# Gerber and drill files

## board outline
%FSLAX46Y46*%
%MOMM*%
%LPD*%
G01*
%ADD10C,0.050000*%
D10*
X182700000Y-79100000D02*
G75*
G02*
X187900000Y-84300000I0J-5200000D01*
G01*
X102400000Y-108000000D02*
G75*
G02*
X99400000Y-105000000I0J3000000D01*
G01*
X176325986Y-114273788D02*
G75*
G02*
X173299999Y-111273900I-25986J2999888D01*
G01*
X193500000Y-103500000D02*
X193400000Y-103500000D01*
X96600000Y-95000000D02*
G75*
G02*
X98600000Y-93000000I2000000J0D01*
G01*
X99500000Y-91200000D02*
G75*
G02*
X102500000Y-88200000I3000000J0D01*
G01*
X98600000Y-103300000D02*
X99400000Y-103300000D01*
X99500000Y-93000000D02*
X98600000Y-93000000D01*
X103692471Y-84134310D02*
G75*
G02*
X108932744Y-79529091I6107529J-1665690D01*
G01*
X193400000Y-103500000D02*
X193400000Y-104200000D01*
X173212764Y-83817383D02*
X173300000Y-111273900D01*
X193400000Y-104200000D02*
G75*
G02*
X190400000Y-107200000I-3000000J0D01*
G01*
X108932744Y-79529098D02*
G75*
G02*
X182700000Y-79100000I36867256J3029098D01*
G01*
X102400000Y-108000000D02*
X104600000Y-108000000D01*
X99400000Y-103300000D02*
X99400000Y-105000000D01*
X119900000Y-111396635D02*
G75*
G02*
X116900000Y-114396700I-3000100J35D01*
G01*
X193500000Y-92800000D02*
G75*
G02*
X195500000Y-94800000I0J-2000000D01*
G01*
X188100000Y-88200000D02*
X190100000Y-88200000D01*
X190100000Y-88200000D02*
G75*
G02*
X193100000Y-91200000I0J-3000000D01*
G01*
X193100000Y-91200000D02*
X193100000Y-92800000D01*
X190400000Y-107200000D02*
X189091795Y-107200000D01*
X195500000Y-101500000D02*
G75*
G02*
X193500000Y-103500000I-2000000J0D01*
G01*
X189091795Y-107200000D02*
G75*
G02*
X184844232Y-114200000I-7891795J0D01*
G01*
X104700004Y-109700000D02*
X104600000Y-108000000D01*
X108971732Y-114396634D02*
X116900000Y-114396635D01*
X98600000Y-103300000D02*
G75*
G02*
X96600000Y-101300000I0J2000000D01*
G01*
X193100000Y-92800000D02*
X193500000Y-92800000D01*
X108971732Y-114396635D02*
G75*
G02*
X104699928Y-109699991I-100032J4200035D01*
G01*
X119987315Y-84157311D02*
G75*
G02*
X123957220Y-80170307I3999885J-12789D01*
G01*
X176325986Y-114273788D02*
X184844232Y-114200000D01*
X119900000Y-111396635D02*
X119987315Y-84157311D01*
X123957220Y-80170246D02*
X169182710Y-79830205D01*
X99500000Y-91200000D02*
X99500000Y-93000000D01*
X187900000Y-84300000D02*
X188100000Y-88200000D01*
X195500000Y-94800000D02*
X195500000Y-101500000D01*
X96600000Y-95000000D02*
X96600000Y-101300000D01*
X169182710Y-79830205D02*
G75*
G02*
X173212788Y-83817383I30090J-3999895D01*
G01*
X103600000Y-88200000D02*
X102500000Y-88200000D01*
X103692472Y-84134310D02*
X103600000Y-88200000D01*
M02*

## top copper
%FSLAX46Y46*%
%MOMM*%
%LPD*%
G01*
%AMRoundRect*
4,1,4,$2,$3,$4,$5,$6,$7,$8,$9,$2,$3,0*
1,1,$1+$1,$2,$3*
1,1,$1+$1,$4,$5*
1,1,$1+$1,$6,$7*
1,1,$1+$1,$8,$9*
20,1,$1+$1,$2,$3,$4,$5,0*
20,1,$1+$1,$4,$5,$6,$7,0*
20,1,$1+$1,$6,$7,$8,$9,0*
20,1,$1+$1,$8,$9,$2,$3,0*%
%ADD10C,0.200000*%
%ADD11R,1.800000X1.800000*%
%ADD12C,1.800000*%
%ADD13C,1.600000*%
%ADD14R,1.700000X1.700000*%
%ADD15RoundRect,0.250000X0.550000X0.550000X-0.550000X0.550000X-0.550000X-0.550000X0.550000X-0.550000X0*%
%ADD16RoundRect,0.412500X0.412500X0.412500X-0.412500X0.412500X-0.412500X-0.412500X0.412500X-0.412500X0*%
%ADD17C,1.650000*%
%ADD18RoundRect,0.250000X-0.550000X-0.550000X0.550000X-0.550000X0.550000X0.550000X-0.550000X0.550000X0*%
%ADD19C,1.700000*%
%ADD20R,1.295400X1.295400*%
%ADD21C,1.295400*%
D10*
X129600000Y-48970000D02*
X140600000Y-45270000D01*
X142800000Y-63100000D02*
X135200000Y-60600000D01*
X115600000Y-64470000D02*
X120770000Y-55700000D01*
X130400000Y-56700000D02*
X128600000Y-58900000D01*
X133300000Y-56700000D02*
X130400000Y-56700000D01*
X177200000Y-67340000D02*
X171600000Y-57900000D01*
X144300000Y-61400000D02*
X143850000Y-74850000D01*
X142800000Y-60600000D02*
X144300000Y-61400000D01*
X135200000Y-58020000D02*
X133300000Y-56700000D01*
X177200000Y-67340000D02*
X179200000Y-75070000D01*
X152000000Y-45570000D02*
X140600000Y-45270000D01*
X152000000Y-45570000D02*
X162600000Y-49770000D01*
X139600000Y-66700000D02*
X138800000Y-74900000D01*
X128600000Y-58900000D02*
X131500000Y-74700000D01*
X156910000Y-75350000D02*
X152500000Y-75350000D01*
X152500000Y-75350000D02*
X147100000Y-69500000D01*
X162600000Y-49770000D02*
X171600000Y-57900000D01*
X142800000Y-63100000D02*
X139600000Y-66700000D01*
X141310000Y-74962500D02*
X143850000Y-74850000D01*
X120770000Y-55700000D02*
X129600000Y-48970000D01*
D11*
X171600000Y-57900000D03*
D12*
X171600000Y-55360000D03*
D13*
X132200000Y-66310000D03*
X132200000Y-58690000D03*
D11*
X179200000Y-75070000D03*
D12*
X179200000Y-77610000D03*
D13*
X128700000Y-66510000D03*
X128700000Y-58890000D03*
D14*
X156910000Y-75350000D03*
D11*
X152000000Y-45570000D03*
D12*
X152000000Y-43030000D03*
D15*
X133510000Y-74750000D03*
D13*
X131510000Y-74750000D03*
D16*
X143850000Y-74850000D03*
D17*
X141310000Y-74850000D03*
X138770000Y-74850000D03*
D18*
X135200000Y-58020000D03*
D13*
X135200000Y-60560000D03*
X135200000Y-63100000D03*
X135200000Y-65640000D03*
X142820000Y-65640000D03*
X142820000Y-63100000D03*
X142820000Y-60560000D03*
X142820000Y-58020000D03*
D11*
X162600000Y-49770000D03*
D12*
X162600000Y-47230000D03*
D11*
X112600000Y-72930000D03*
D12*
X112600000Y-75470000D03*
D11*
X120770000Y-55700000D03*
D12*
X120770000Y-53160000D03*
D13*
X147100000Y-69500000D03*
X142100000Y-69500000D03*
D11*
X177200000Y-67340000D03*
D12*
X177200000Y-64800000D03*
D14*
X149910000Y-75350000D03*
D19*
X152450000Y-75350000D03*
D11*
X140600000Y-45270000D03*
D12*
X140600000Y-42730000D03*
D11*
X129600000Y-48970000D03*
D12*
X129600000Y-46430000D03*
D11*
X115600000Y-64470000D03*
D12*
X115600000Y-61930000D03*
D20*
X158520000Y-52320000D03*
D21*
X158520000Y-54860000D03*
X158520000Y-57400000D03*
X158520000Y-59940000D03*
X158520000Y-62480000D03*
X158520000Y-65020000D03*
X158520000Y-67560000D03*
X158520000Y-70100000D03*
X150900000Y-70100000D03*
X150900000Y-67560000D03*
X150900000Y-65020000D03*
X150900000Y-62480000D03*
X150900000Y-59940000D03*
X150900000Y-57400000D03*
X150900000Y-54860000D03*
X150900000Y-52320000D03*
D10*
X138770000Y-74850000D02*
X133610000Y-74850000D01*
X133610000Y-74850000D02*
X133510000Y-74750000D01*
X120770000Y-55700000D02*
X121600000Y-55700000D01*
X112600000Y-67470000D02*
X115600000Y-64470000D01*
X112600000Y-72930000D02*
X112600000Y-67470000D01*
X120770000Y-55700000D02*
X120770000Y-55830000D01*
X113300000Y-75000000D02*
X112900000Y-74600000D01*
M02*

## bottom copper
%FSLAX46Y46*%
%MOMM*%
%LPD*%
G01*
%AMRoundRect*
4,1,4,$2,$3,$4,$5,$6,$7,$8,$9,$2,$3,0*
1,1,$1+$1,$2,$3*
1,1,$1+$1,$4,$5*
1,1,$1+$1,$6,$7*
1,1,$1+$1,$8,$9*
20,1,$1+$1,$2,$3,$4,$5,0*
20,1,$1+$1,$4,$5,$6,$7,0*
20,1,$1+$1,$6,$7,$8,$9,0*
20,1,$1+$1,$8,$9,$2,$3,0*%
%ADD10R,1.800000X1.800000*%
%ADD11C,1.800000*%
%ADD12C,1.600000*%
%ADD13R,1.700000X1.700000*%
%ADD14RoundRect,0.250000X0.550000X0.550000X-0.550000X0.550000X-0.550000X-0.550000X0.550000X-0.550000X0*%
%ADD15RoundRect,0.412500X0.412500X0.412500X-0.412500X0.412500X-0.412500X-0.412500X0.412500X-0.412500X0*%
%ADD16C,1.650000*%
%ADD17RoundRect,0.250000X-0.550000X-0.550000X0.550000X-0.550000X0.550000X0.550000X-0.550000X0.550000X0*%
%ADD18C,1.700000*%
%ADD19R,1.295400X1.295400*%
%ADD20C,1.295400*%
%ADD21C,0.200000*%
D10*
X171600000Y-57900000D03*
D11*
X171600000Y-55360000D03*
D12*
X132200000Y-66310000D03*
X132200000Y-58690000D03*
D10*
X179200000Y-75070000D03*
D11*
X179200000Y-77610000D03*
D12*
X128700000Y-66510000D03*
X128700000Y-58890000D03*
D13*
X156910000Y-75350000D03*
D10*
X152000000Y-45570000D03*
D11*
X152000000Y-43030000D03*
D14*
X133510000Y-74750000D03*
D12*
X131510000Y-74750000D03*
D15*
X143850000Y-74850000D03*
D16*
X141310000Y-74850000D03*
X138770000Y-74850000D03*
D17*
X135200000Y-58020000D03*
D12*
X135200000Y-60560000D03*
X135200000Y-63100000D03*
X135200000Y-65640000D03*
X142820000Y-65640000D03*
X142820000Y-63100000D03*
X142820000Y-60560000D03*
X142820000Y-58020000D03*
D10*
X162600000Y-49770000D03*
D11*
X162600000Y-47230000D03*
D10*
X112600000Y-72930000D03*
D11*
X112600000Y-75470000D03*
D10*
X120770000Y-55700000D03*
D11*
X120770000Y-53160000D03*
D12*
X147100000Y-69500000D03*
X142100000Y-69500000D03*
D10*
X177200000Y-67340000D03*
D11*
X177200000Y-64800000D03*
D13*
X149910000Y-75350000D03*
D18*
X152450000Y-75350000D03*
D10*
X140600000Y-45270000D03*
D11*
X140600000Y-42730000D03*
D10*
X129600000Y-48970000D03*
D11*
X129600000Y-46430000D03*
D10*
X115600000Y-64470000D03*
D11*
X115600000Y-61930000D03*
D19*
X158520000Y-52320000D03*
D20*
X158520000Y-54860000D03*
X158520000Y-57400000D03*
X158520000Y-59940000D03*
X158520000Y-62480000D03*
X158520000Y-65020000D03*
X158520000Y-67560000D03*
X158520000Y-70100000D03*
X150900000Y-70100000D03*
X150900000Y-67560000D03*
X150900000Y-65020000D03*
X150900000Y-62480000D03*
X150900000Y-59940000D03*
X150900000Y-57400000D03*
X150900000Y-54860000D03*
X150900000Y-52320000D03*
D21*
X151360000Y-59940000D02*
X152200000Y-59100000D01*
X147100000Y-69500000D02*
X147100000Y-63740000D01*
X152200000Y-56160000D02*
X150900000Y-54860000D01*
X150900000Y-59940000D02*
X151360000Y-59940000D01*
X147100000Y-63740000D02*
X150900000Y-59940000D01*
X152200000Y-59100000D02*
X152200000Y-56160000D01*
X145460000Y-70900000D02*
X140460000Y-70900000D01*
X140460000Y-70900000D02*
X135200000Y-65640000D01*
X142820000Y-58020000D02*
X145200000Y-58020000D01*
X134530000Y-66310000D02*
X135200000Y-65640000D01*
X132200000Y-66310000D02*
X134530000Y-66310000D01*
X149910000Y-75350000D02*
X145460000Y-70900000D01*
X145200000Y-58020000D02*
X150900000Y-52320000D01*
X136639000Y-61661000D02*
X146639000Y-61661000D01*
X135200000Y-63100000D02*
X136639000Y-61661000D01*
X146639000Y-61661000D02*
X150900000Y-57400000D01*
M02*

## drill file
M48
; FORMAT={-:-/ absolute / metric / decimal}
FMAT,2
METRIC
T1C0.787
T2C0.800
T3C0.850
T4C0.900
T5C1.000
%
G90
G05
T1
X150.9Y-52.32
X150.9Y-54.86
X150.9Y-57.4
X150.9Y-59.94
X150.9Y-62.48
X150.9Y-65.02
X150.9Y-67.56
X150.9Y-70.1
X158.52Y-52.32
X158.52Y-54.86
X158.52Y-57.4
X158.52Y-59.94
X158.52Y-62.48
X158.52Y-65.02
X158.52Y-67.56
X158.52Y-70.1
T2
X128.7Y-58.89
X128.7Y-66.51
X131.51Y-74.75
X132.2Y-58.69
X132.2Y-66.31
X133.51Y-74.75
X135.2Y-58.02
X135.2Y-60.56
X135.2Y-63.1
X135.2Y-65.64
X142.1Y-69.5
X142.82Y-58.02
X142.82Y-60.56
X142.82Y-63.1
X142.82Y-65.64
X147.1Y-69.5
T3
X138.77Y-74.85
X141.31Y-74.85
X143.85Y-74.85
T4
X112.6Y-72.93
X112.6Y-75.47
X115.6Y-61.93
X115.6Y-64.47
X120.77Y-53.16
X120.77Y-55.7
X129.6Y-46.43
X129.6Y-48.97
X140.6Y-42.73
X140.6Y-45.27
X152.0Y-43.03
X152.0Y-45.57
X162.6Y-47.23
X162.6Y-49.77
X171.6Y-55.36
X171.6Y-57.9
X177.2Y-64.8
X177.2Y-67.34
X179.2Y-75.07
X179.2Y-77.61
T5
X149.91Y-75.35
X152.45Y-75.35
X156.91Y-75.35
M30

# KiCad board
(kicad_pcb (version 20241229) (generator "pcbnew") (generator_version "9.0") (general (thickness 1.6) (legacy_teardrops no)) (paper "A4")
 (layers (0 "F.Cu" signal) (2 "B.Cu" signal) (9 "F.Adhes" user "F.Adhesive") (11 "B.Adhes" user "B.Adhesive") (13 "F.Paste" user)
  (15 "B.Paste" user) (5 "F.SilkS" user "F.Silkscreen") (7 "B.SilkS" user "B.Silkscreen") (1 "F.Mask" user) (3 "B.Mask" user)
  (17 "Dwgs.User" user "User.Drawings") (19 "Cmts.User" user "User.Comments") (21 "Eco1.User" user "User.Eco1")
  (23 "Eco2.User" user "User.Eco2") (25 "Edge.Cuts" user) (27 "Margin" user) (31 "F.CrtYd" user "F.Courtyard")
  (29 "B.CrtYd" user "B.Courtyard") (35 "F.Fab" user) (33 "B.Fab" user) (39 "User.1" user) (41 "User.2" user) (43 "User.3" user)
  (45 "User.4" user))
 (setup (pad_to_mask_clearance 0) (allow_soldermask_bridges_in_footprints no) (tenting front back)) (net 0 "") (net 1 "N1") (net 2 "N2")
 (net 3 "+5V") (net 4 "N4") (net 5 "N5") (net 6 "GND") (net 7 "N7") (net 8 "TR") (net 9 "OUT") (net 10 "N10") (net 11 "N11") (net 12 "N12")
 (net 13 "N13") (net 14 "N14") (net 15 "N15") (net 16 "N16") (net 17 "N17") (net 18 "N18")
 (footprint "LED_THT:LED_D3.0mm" (layer "F.Cu") (at 171.6 57.9 90)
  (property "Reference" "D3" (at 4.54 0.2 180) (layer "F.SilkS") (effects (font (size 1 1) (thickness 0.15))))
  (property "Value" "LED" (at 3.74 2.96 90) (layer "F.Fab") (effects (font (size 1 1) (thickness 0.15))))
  (pad "1" thru_hole rect (at 0 0 90) (size 1.8 1.8) (drill 0.9) (layers "*.Cu" "*.Mask") (remove_unused_layers no) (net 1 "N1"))
  (pad "2" thru_hole circle (at 2.54 0 90) (size 1.8 1.8) (drill 0.9) (layers "*.Cu" "*.Mask") (remove_unused_layers no) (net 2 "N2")))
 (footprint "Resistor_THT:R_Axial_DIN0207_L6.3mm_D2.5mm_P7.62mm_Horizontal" (layer "F.Cu") (at 132.2 66.31 90)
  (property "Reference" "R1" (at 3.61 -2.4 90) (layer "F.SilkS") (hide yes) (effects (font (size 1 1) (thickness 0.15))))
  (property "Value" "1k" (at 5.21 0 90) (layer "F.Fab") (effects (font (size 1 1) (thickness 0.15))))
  (pad "1" thru_hole circle (at 0 0 90) (size 1.6 1.6) (drill 0.8) (layers "*.Cu" "*.Mask") (remove_unused_layers no) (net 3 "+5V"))
  (pad "2" thru_hole circle (at 7.62 0 90) (size 1.6 1.6) (drill 0.8) (layers "*.Cu" "*.Mask") (remove_unused_layers no) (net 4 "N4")))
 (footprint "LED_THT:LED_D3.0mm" (layer "F.Cu") (at 179.2 75.07 -90)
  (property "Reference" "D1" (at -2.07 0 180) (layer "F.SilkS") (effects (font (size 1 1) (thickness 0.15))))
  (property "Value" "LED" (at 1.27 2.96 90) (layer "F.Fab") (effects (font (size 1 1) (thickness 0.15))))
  (pad "1" thru_hole rect (at 0 0 270) (size 1.8 1.8) (drill 0.9) (layers "*.Cu" "*.Mask") (remove_unused_layers no) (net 1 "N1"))
  (pad "2" thru_hole circle (at 2.54 0 270) (size 1.8 1.8) (drill 0.9) (layers "*.Cu" "*.Mask") (remove_unused_layers no) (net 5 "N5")))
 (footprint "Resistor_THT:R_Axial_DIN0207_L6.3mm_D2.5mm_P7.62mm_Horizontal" (layer "F.Cu") (at 128.7 66.51 90)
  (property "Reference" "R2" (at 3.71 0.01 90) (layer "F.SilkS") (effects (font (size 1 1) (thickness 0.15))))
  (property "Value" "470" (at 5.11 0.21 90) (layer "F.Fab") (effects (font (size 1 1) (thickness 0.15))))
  (pad "1" thru_hole circle (at 0 0 90) (size 1.6 1.6) (drill 0.8) (layers "*.Cu" "*.Mask") (remove_unused_layers no) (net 1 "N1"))
  (pad "2" thru_hole circle (at 7.62 0 90) (size 1.6 1.6) (drill 0.8) (layers "*.Cu" "*.Mask") (remove_unused_layers no) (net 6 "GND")))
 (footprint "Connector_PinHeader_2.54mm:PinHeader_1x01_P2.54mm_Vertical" (layer "F.Cu") (at 156.91 75.35)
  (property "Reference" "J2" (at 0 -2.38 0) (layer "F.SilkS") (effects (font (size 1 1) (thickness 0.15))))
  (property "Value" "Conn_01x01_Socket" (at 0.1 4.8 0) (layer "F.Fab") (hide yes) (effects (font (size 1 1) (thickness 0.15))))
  (pad "1" thru_hole rect (at 0 0) (size 1.7 1.7) (drill 1) (layers "*.Cu" "*.Mask") (remove_unused_layers no) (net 6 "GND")))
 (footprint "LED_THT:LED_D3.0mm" (layer "F.Cu") (at 152 45.57 90)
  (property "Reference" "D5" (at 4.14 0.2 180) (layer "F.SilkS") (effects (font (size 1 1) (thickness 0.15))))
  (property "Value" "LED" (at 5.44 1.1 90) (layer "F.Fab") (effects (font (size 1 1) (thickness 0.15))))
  (pad "1" thru_hole rect (at 0 0 90) (size 1.8 1.8) (drill 0.9) (layers "*.Cu" "*.Mask") (remove_unused_layers no) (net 1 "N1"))
  (pad "2" thru_hole circle (at 2.54 0 90) (size 1.8 1.8) (drill 0.9) (layers "*.Cu" "*.Mask") (remove_unused_layers no) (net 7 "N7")))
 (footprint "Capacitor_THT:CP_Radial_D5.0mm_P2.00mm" (layer "F.Cu") (at 133.51 74.75 180)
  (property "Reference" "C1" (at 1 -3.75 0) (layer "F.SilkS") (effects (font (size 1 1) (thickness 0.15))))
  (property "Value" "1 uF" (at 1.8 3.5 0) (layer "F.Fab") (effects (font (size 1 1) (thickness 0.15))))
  (pad "1" thru_hole roundrect (at 0 0 180) (size 1.6 1.6) (drill 0.8) (layers "*.Cu" "*.Mask") (remove_unused_layers no)
   (roundrect_rratio 0.15625) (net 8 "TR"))
  (pad "2" thru_hole circle (at 2 0 180) (size 1.6 1.6) (drill 0.8) (layers "*.Cu" "*.Mask") (remove_unused_layers no) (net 6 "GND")))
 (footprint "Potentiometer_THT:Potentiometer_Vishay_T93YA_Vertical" (layer "F.Cu") (at 143.85 74.85 180)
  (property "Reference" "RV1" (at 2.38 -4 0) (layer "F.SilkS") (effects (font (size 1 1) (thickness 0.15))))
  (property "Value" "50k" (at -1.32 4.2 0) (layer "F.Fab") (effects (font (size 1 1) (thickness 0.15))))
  (pad "1" thru_hole roundrect (at 0 0 180) (size 1.65 1.65) (drill 0.85) (layers "*.Cu" "*.Mask") (remove_unused_layers no)
   (roundrect_rratio 0.25) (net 4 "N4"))
  (pad "2" thru_hole circle (at 2.54 0 180) (size 1.65 1.65) (drill 0.85) (layers "*.Cu" "*.Mask") (remove_unused_layers no) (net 4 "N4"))
  (pad "3" thru_hole circle (at 5.08 0 180) (size 1.65 1.65) (drill 0.85) (layers "*.Cu" "*.Mask") (remove_unused_layers no) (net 8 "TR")))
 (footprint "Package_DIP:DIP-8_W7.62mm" (layer "F.Cu") (at 135.2 58.02)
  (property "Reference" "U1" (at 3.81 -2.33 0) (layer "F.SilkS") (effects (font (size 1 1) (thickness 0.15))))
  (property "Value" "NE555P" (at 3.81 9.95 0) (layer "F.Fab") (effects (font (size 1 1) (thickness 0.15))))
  (pad "1" thru_hole roundrect (at 0 0) (size 1.6 1.6) (drill 0.8) (layers "*.Cu" "*.Mask") (remove_unused_layers no)
   (roundrect_rratio 0.15625) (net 6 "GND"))
  (pad "2" thru_hole circle (at 0 2.54) (size 1.6 1.6) (drill 0.8) (layers "*.Cu" "*.Mask") (remove_unused_layers no) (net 8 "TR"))
  (pad "3" thru_hole circle (at 0 5.08) (size 1.6 1.6) (drill 0.8) (layers "*.Cu" "*.Mask") (remove_unused_layers no) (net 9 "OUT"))
  (pad "4" thru_hole circle (at 0 7.62) (size 1.6 1.6) (drill 0.8) (layers "*.Cu" "*.Mask") (remove_unused_layers no) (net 3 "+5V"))
  (pad "5" thru_hole circle (at 7.62 7.62) (size 1.6 1.6) (drill 0.8) (layers "*.Cu" "*.Mask") (remove_unused_layers no) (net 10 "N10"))
  (pad "6" thru_hole circle (at 7.62 5.08) (size 1.6 1.6) (drill 0.8) (layers "*.Cu" "*.Mask") (remove_unused_layers no) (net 8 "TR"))
  (pad "7" thru_hole circle (at 7.62 2.54) (size 1.6 1.6) (drill 0.8) (layers "*.Cu" "*.Mask") (remove_unused_layers no) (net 4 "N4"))
  (pad "8" thru_hole circle (at 7.62 0) (size 1.6 1.6) (drill 0.8) (layers "*.Cu" "*.Mask") (remove_unused_layers no) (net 3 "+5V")))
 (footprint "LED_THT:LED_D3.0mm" (layer "F.Cu") (at 162.6 49.77 90)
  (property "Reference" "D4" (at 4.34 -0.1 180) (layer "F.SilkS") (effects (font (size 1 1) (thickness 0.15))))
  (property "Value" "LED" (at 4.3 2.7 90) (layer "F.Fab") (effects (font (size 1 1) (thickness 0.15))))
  (pad "1" thru_hole rect (at 0 0 90) (size 1.8 1.8) (drill 0.9) (layers "*.Cu" "*.Mask") (remove_unused_layers no) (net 1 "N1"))
  (pad "2" thru_hole circle (at 2.54 0 90) (size 1.8 1.8) (drill 0.9) (layers "*.Cu" "*.Mask") (remove_unused_layers no) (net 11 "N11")))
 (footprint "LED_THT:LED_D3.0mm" (layer "F.Cu") (at 112.6 72.93 -90)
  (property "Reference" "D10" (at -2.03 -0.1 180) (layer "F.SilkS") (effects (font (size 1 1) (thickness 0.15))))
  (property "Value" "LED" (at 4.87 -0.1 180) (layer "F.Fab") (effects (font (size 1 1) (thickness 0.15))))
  (pad "1" thru_hole rect (at 0 0 270) (size 1.8 1.8) (drill 0.9) (layers "*.Cu" "*.Mask") (remove_unused_layers no) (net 1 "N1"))
  (pad "2" thru_hole circle (at 2.54 0 270) (size 1.8 1.8) (drill 0.9) (layers "*.Cu" "*.Mask") (remove_unused_layers no) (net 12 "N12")))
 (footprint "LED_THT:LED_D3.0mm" (layer "F.Cu") (at 120.77 55.7 90)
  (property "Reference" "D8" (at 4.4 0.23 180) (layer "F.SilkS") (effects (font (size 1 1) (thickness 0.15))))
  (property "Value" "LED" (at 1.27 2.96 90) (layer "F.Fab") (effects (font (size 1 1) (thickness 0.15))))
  (pad "1" thru_hole rect (at 0 0 90) (size 1.8 1.8) (drill 0.9) (layers "*.Cu" "*.Mask") (remove_unused_layers no) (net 1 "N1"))
  (pad "2" thru_hole circle (at 2.54 0 90) (size 1.8 1.8) (drill 0.9) (layers "*.Cu" "*.Mask") (remove_unused_layers no) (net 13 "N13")))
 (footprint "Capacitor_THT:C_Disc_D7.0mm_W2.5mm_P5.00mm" (layer "F.Cu") (at 147.1 69.5 180)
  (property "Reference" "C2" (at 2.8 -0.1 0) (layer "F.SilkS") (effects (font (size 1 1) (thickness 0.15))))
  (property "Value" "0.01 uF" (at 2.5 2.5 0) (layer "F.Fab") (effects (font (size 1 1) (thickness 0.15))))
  (pad "1" thru_hole circle (at 0 0 180) (size 1.6 1.6) (drill 0.8) (layers "*.Cu" "*.Mask") (remove_unused_layers no) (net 6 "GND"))
  (pad "2" thru_hole circle (at 5 0 180) (size 1.6 1.6) (drill 0.8) (layers "*.Cu" "*.Mask") (remove_unused_layers no) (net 10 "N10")))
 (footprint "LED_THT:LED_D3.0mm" (layer "F.Cu") (at 177.2 67.34 90)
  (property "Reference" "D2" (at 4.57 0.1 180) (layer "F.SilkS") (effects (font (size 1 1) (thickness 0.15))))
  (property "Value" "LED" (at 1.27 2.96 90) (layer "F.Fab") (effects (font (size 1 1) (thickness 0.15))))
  (pad "1" thru_hole rect (at 0 0 90) (size 1.8 1.8) (drill 0.9) (layers "*.Cu" "*.Mask") (remove_unused_layers no) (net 1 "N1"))
  (pad "2" thru_hole circle (at 2.54 0 90) (size 1.8 1.8) (drill 0.9) (layers "*.Cu" "*.Mask") (remove_unused_layers no) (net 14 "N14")))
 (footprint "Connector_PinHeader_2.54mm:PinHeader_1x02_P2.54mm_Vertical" (layer "F.Cu") (at 149.91 75.35 90)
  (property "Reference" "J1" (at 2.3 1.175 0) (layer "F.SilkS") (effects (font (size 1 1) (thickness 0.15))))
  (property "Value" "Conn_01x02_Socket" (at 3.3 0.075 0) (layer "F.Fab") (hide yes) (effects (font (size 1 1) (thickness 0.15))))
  (pad "1" thru_hole rect (at 0 0 90) (size 1.7 1.7) (drill 1) (layers "*.Cu" "*.Mask") (remove_unused_layers no) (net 3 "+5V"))
  (pad "2" thru_hole circle (at 0 2.54 90) (size 1.7 1.7) (drill 1) (layers "*.Cu" "*.Mask") (remove_unused_layers no) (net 6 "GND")))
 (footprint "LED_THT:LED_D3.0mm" (layer "F.Cu") (at 140.6 45.27 90)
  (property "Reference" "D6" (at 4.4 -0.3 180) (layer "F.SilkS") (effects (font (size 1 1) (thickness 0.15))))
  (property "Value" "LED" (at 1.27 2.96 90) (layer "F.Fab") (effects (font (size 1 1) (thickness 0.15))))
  (pad "1" thru_hole rect (at 0 0 90) (size 1.8 1.8) (drill 0.9) (layers "*.Cu" "*.Mask") (remove_unused_layers no) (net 1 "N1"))
  (pad "2" thru_hole circle (at 2.54 0 90) (size 1.8 1.8) (drill 0.9) (layers "*.Cu" "*.Mask") (remove_unused_layers no) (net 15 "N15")))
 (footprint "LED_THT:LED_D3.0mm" (layer "F.Cu") (at 129.6 48.97 90)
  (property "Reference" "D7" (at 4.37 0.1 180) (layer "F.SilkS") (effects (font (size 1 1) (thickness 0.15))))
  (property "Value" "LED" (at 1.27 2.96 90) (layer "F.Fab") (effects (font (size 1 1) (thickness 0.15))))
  (pad "1" thru_hole rect (at 0 0 90) (size 1.8 1.8) (drill 0.9) (layers "*.Cu" "*.Mask") (remove_unused_layers no) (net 1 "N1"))
  (pad "2" thru_hole circle (at 2.54 0 90) (size 1.8 1.8) (drill 0.9) (layers "*.Cu" "*.Mask") (remove_unused_layers no) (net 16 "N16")))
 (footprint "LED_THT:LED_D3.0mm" (layer "F.Cu") (at 115.6 64.47 90)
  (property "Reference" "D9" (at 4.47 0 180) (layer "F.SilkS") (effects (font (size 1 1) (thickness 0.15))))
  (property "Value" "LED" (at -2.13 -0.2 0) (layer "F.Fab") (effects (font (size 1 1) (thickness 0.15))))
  (pad "1" thru_hole rect (at 0 0 90) (size 1.8 1.8) (drill 0.9) (layers "*.Cu" "*.Mask") (remove_unused_layers no) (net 1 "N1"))
  (pad "2" thru_hole circle (at 2.54 0 90) (size 1.8 1.8) (drill 0.9) (layers "*.Cu" "*.Mask") (remove_unused_layers no) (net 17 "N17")))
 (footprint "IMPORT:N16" (layer "B.Cu") (at 150.9 70.1 180)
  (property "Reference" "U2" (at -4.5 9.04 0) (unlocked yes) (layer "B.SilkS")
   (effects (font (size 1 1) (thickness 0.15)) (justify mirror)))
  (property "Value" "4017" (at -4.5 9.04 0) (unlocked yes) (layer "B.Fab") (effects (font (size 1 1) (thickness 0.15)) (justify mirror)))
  (pad "1" thru_hole rect (at -7.62 17.78 180) (size 1.2954 1.2954) (drill 0.7874) (layers "*.Cu" "*.Mask") (remove_unused_layers no)
   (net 15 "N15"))
  (pad "2" thru_hole circle (at -7.62 15.24 180) (size 1.2954 1.2954) (drill 0.7874) (layers "*.Cu" "*.Mask") (remove_unused_layers no)
   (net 14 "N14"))
  (pad "3" thru_hole circle (at -7.62 12.7 180) (size 1.2954 1.2954) (drill 0.7874) (layers "*.Cu" "*.Mask") (remove_unused_layers no)
   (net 5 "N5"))
  (pad "4" thru_hole circle (at -7.62 10.16 180) (size 1.2954 1.2954) (drill 0.7874) (layers "*.Cu" "*.Mask") (remove_unused_layers no)
   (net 2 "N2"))
  (pad "5" thru_hole circle (at -7.62 7.62 180) (size 1.2954 1.2954) (drill 0.7874) (layers "*.Cu" "*.Mask") (remove_unused_layers no)
   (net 16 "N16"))
  (pad "6" thru_hole circle (at -7.62 5.08 180) (size 1.2954 1.2954) (drill 0.7874) (layers "*.Cu" "*.Mask") (remove_unused_layers no)
   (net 13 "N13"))
  (pad "7" thru_hole circle (at -7.62 2.54 180) (size 1.2954 1.2954) (drill 0.7874) (layers "*.Cu" "*.Mask") (remove_unused_layers no)
   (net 11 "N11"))
  (pad "8" thru_hole circle (at -7.62 0 180) (size 1.2954 1.2954) (drill 0.7874) (layers "*.Cu" "*.Mask") (remove_unused_layers no)
   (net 6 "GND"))
  (pad "9" thru_hole circle (at 0 0 180) (size 1.2954 1.2954) (drill 0.7874) (layers "*.Cu" "*.Mask") (remove_unused_layers no)
   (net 17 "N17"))
  (pad "10" thru_hole circle (at 0 2.54 180) (size 1.2954 1.2954) (drill 0.7874) (layers "*.Cu" "*.Mask") (remove_unused_layers no)
   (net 7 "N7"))
  (pad "11" thru_hole circle (at 0 5.08 180) (size 1.2954 1.2954) (drill 0.7874) (layers "*.Cu" "*.Mask") (remove_unused_layers no)
   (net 12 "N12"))
  (pad "12" thru_hole circle (at 0 7.62 180) (size 1.2954 1.2954) (drill 0.7874) (layers "*.Cu" "*.Mask") (remove_unused_layers no)
   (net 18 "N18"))
  (pad "13" thru_hole circle (at 0 10.16 180) (size 1.2954 1.2954) (drill 0.7874) (layers "*.Cu" "*.Mask") (remove_unused_layers no)
   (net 6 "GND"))
  (pad "14" thru_hole circle (at 0 12.7 180) (size 1.2954 1.2954) (drill 0.7874) (layers "*.Cu" "*.Mask") (remove_unused_layers no)
   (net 9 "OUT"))
  (pad "15" thru_hole circle (at 0 15.24 180) (size 1.2954 1.2954) (drill 0.7874) (layers "*.Cu" "*.Mask") (remove_unused_layers no)
   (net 6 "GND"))
  (pad "16" thru_hole circle (at 0 17.78 180) (size 1.2954 1.2954) (drill 0.7874) (layers "*.Cu" "*.Mask") (remove_unused_layers no)
   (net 3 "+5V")))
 (gr_line (start 129.6 48.97) (end 140.6 45.27) (stroke (width 0.2) (type default)) (layer "F.Cu") (net 1))
 (gr_line (start 142.8 63.1) (end 135.2 60.6) (stroke (width 0.2) (type default)) (layer "F.Cu") (net 8))
 (gr_line (start 115.6 64.47) (end 120.77 55.7) (stroke (width 0.2) (type default)) (layer "F.Cu") (net 1))
 (gr_line (start 130.4 56.7) (end 128.6 58.9) (stroke (width 0.2) (type default)) (layer "F.Cu") (net 6))
 (gr_line (start 133.3 56.7) (end 130.4 56.7) (stroke (width 0.2) (type default)) (layer "F.Cu") (net 6))
 (gr_line (start 177.2 67.34) (end 171.6 57.9) (stroke (width 0.2) (type default)) (layer "F.Cu") (net 1))
 (gr_line (start 144.3 61.4) (end 143.85 74.85) (stroke (width 0.2) (type default)) (layer "F.Cu") (net 4))
 (gr_line (start 142.8 60.6) (end 144.3 61.4) (stroke (width 0.2) (type default)) (layer "F.Cu") (net 4))
 (gr_line (start 135.2 58.02) (end 133.3 56.7) (stroke (width 0.2) (type default)) (layer "F.Cu") (net 6))
 (gr_line (start 177.2 67.34) (end 179.2 75.07) (stroke (width 0.2) (type default)) (layer "F.Cu") (net 1))
 (gr_line (start 152 45.57) (end 140.6 45.27) (stroke (width 0.2) (type default)) (layer "F.Cu") (net 1))
 (gr_line (start 152 45.57) (end 162.6 49.77) (stroke (width 0.2) (type default)) (layer "F.Cu") (net 1))
 (gr_line (start 139.6 66.7) (end 138.8 74.9) (stroke (width 0.2) (type default)) (layer "F.Cu") (net 8))
 (gr_line (start 128.6 58.9) (end 131.5 74.7) (stroke (width 0.2) (type default)) (layer "F.Cu") (net 6))
 (gr_line (start 156.91 75.35) (end 152.5 75.35) (stroke (width 0.2) (type default)) (layer "F.Cu") (net 6))
 (gr_line (start 152.5 75.35) (end 147.1 69.5) (stroke (width 0.2) (type default)) (layer "F.Cu") (net 6))
 (gr_line (start 162.6 49.77) (end 171.6 57.9) (stroke (width 0.2) (type default)) (layer "F.Cu") (net 1))
 (gr_line (start 142.8 63.1) (end 139.6 66.7) (stroke (width 0.2) (type default)) (layer "F.Cu") (net 8))
 (gr_line (start 141.31 74.9625) (end 143.85 74.85) (stroke (width 0.2) (type default)) (layer "F.Cu") (net 4))
 (gr_line (start 120.77 55.7) (end 129.6 48.97) (stroke (width 0.2) (type default)) (layer "F.Cu") (net 1))
 (gr_arc (start 182.7 79.1) (mid 186.376955 80.623045) (end 187.9 84.3) (stroke (width 0.05) (type default)) (layer "Edge.Cuts"))
 (gr_arc (start 102.4 108) (mid 100.27868 107.12132) (end 99.4 105) (stroke (width 0.05) (type default)) (layer "Edge.Cuts"))
 (gr_arc (start 176.325986 114.273788) (mid 174.187887 113.404388) (end 173.3 111.2739) (stroke (width 0.05) (type default))
  (layer "Edge.Cuts"))
 (gr_line (start 193.5 103.5) (end 193.4 103.5) (stroke (width 0.05) (type default)) (layer "Edge.Cuts"))
 (gr_arc (start 96.6 95) (mid 97.185786 93.585786) (end 98.6 93) (stroke (width 0.05) (type default)) (layer "Edge.Cuts"))
 (gr_arc (start 99.5 91.2) (mid 100.37868 89.07868) (end 102.5 88.2) (stroke (width 0.05) (type default)) (layer "Edge.Cuts"))
 (gr_line (start 98.6 103.3) (end 99.4 103.3) (stroke (width 0.05) (type default)) (layer "Edge.Cuts"))
 (gr_line (start 99.5 93) (end 98.6 93) (stroke (width 0.05) (type default)) (layer "Edge.Cuts"))
 (gr_arc (start 103.692471 84.13431) (mid 105.621015 81.044738) (end 108.932744 79.529091) (stroke (width 0.05) (type default))
  (layer "Edge.Cuts"))
 (gr_line (start 193.4 103.5) (end 193.4 104.2) (stroke (width 0.05) (type default)) (layer "Edge.Cuts"))
 (gr_line (start 173.212764 83.817383) (end 173.3 111.2739) (stroke (width 0.05) (type default)) (layer "Edge.Cuts"))
 (gr_arc (start 193.4 104.2) (mid 192.52132 106.32132) (end 190.4 107.2) (stroke (width 0.05) (type default)) (layer "Edge.Cuts"))
 (gr_arc (start 108.932744 79.529098) (mid 145.584827 39.50914) (end 182.7 79.1) (stroke (width 0.05) (type default)) (layer "Edge.Cuts"))
 (gr_line (start 102.4 108) (end 104.6 108) (stroke (width 0.05) (type default)) (layer "Edge.Cuts"))
 (gr_line (start 99.4 103.3) (end 99.4 105) (stroke (width 0.05) (type default)) (layer "Edge.Cuts"))
 (gr_arc (start 119.9 111.396635) (mid 119.021308 113.517933) (end 116.9 114.396635) (stroke (width 0.05) (type default))
  (layer "Edge.Cuts"))
 (gr_arc (start 193.5 92.8) (mid 194.914214 93.385786) (end 195.5 94.8) (stroke (width 0.05) (type default)) (layer "Edge.Cuts"))
 (gr_line (start 188.1 88.2) (end 190.1 88.2) (stroke (width 0.05) (type default)) (layer "Edge.Cuts"))
 (gr_arc (start 190.1 88.2) (mid 192.22132 89.07868) (end 193.1 91.2) (stroke (width 0.05) (type default)) (layer "Edge.Cuts"))
 (gr_line (start 193.1 91.2) (end 193.1 92.8) (stroke (width 0.05) (type default)) (layer "Edge.Cuts"))
 (gr_line (start 190.4 107.2) (end 189.091795 107.2) (stroke (width 0.05) (type default)) (layer "Edge.Cuts"))
 (gr_arc (start 195.5 101.5) (mid 194.914214 102.914214) (end 193.5 103.5) (stroke (width 0.05) (type default)) (layer "Edge.Cuts"))
 (gr_arc (start 189.091795 107.2) (mid 187.94685 111.293953) (end 184.844232 114.2) (stroke (width 0.05) (type default)) (layer "Edge.Cuts"))
 (gr_line (start 104.700004 109.7) (end 104.6 108) (stroke (width 0.05) (type default)) (layer "Edge.Cuts"))
 (gr_line (start 108.971732 114.396634) (end 116.9 114.396635) (stroke (width 0.05) (type default)) (layer "Edge.Cuts"))
 (gr_arc (start 98.6 103.3) (mid 97.185786 102.714214) (end 96.6 101.3) (stroke (width 0.05) (type default)) (layer "Edge.Cuts"))
 (gr_line (start 193.1 92.8) (end 193.5 92.8) (stroke (width 0.05) (type default)) (layer "Edge.Cuts"))
 (gr_arc (start 108.971732 114.396635) (mid 105.763783 113.023409) (end 104.7 109.7) (stroke (width 0.05) (type default))
  (layer "Edge.Cuts"))
 (gr_arc (start 119.987315 84.157311) (mid 121.152762 81.347789) (end 123.95722 80.170246) (stroke (width 0.05) (type default))
  (layer "Edge.Cuts"))
 (gr_line (start 176.325986 114.273788) (end 184.844232 114.2) (stroke (width 0.05) (type default)) (layer "Edge.Cuts"))
 (gr_line (start 119.9 111.396635) (end 119.987315 84.157311) (stroke (width 0.05) (type default)) (layer "Edge.Cuts"))
 (gr_line (start 123.95722 80.170246) (end 169.18271 79.830205) (stroke (width 0.05) (type default)) (layer "Edge.Cuts"))
 (gr_line (start 99.5 91.2) (end 99.5 93) (stroke (width 0.05) (type default)) (layer "Edge.Cuts"))
 (gr_line (start 187.9 84.3) (end 188.1 88.2) (stroke (width 0.05) (type default)) (layer "Edge.Cuts"))
 (gr_line (start 195.5 94.8) (end 195.5 101.5) (stroke (width 0.05) (type default)) (layer "Edge.Cuts"))
 (gr_line (start 96.6 95) (end 96.6 101.3) (stroke (width 0.05) (type default)) (layer "Edge.Cuts"))
 (gr_arc (start 169.18271 79.830205) (mid 172.026045 80.986579) (end 173.212764 83.817383) (stroke (width 0.05) (type default))
  (layer "Edge.Cuts"))
 (gr_line (start 103.6 88.2) (end 102.5 88.2) (stroke (width 0.05) (type default)) (layer "Edge.Cuts"))
 (gr_line (start 103.692472 84.13431) (end 103.6 88.2) (stroke (width 0.05) (type default)) (layer "Edge.Cuts"))
 (segment (start 138.77 74.85) (end 133.61 74.85) (width 0.2) (layer "F.Cu") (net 8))
 (segment (start 133.61 74.85) (end 133.51 74.75) (width 0.2) (layer "F.Cu") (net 8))
 (segment (start 151.36 59.94) (end 152.2 59.1) (width 0.2) (layer "B.Cu") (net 6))
 (segment (start 147.1 69.5) (end 147.1 63.74) (width 0.2) (layer "B.Cu") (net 6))
 (segment (start 152.2 56.16) (end 150.9 54.86) (width 0.2) (layer "B.Cu") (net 6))
 (segment (start 150.9 59.94) (end 151.36 59.94) (width 0.2) (layer "B.Cu") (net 6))
 (segment (start 147.1 63.74) (end 150.9 59.94) (width 0.2) (layer "B.Cu") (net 6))
 (segment (start 152.2 59.1) (end 152.2 56.16) (width 0.2) (layer "B.Cu") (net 6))
 (segment (start 120.77 55.7) (end 121.6 55.7) (width 0.2) (layer "F.Cu") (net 1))
 (segment (start 112.6 67.47) (end 115.6 64.47) (width 0.2) (layer "F.Cu") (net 1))
 (segment (start 112.6 72.93) (end 112.6 67.47) (width 0.2) (layer "F.Cu") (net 1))
 (segment (start 120.77 55.7) (end 120.77 55.83) (width 0.2) (layer "F.Cu") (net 1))
 (segment (start 113.3 75) (end 112.9 74.6) (width 0.2) (layer "F.Cu") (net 12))
 (segment (start 145.46 70.9) (end 140.46 70.9) (width 0.2) (layer "B.Cu") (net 3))
 (segment (start 140.46 70.9) (end 135.2 65.64) (width 0.2) (layer "B.Cu") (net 3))
 (segment (start 142.82 58.02) (end 145.2 58.02) (width 0.2) (layer "B.Cu") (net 3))
 (segment (start 134.53 66.31) (end 135.2 65.64) (width 0.2) (layer "B.Cu") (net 3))
 (segment (start 132.2 66.31) (end 134.53 66.31) (width 0.2) (layer "B.Cu") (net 3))
 (segment (start 149.91 75.35) (end 145.46 70.9) (width 0.2) (layer "B.Cu") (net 3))
 (segment (start 145.2 58.02) (end 150.9 52.32) (width 0.2) (layer "B.Cu") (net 3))
 (segment (start 136.639 61.661) (end 146.639 61.661) (width 0.2) (layer "B.Cu") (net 9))
 (segment (start 135.2 63.1) (end 136.639 61.661) (width 0.2) (layer "B.Cu") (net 9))
 (segment (start 146.639 61.661) (end 150.9 57.4) (width 0.2) (layer "B.Cu") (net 9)))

